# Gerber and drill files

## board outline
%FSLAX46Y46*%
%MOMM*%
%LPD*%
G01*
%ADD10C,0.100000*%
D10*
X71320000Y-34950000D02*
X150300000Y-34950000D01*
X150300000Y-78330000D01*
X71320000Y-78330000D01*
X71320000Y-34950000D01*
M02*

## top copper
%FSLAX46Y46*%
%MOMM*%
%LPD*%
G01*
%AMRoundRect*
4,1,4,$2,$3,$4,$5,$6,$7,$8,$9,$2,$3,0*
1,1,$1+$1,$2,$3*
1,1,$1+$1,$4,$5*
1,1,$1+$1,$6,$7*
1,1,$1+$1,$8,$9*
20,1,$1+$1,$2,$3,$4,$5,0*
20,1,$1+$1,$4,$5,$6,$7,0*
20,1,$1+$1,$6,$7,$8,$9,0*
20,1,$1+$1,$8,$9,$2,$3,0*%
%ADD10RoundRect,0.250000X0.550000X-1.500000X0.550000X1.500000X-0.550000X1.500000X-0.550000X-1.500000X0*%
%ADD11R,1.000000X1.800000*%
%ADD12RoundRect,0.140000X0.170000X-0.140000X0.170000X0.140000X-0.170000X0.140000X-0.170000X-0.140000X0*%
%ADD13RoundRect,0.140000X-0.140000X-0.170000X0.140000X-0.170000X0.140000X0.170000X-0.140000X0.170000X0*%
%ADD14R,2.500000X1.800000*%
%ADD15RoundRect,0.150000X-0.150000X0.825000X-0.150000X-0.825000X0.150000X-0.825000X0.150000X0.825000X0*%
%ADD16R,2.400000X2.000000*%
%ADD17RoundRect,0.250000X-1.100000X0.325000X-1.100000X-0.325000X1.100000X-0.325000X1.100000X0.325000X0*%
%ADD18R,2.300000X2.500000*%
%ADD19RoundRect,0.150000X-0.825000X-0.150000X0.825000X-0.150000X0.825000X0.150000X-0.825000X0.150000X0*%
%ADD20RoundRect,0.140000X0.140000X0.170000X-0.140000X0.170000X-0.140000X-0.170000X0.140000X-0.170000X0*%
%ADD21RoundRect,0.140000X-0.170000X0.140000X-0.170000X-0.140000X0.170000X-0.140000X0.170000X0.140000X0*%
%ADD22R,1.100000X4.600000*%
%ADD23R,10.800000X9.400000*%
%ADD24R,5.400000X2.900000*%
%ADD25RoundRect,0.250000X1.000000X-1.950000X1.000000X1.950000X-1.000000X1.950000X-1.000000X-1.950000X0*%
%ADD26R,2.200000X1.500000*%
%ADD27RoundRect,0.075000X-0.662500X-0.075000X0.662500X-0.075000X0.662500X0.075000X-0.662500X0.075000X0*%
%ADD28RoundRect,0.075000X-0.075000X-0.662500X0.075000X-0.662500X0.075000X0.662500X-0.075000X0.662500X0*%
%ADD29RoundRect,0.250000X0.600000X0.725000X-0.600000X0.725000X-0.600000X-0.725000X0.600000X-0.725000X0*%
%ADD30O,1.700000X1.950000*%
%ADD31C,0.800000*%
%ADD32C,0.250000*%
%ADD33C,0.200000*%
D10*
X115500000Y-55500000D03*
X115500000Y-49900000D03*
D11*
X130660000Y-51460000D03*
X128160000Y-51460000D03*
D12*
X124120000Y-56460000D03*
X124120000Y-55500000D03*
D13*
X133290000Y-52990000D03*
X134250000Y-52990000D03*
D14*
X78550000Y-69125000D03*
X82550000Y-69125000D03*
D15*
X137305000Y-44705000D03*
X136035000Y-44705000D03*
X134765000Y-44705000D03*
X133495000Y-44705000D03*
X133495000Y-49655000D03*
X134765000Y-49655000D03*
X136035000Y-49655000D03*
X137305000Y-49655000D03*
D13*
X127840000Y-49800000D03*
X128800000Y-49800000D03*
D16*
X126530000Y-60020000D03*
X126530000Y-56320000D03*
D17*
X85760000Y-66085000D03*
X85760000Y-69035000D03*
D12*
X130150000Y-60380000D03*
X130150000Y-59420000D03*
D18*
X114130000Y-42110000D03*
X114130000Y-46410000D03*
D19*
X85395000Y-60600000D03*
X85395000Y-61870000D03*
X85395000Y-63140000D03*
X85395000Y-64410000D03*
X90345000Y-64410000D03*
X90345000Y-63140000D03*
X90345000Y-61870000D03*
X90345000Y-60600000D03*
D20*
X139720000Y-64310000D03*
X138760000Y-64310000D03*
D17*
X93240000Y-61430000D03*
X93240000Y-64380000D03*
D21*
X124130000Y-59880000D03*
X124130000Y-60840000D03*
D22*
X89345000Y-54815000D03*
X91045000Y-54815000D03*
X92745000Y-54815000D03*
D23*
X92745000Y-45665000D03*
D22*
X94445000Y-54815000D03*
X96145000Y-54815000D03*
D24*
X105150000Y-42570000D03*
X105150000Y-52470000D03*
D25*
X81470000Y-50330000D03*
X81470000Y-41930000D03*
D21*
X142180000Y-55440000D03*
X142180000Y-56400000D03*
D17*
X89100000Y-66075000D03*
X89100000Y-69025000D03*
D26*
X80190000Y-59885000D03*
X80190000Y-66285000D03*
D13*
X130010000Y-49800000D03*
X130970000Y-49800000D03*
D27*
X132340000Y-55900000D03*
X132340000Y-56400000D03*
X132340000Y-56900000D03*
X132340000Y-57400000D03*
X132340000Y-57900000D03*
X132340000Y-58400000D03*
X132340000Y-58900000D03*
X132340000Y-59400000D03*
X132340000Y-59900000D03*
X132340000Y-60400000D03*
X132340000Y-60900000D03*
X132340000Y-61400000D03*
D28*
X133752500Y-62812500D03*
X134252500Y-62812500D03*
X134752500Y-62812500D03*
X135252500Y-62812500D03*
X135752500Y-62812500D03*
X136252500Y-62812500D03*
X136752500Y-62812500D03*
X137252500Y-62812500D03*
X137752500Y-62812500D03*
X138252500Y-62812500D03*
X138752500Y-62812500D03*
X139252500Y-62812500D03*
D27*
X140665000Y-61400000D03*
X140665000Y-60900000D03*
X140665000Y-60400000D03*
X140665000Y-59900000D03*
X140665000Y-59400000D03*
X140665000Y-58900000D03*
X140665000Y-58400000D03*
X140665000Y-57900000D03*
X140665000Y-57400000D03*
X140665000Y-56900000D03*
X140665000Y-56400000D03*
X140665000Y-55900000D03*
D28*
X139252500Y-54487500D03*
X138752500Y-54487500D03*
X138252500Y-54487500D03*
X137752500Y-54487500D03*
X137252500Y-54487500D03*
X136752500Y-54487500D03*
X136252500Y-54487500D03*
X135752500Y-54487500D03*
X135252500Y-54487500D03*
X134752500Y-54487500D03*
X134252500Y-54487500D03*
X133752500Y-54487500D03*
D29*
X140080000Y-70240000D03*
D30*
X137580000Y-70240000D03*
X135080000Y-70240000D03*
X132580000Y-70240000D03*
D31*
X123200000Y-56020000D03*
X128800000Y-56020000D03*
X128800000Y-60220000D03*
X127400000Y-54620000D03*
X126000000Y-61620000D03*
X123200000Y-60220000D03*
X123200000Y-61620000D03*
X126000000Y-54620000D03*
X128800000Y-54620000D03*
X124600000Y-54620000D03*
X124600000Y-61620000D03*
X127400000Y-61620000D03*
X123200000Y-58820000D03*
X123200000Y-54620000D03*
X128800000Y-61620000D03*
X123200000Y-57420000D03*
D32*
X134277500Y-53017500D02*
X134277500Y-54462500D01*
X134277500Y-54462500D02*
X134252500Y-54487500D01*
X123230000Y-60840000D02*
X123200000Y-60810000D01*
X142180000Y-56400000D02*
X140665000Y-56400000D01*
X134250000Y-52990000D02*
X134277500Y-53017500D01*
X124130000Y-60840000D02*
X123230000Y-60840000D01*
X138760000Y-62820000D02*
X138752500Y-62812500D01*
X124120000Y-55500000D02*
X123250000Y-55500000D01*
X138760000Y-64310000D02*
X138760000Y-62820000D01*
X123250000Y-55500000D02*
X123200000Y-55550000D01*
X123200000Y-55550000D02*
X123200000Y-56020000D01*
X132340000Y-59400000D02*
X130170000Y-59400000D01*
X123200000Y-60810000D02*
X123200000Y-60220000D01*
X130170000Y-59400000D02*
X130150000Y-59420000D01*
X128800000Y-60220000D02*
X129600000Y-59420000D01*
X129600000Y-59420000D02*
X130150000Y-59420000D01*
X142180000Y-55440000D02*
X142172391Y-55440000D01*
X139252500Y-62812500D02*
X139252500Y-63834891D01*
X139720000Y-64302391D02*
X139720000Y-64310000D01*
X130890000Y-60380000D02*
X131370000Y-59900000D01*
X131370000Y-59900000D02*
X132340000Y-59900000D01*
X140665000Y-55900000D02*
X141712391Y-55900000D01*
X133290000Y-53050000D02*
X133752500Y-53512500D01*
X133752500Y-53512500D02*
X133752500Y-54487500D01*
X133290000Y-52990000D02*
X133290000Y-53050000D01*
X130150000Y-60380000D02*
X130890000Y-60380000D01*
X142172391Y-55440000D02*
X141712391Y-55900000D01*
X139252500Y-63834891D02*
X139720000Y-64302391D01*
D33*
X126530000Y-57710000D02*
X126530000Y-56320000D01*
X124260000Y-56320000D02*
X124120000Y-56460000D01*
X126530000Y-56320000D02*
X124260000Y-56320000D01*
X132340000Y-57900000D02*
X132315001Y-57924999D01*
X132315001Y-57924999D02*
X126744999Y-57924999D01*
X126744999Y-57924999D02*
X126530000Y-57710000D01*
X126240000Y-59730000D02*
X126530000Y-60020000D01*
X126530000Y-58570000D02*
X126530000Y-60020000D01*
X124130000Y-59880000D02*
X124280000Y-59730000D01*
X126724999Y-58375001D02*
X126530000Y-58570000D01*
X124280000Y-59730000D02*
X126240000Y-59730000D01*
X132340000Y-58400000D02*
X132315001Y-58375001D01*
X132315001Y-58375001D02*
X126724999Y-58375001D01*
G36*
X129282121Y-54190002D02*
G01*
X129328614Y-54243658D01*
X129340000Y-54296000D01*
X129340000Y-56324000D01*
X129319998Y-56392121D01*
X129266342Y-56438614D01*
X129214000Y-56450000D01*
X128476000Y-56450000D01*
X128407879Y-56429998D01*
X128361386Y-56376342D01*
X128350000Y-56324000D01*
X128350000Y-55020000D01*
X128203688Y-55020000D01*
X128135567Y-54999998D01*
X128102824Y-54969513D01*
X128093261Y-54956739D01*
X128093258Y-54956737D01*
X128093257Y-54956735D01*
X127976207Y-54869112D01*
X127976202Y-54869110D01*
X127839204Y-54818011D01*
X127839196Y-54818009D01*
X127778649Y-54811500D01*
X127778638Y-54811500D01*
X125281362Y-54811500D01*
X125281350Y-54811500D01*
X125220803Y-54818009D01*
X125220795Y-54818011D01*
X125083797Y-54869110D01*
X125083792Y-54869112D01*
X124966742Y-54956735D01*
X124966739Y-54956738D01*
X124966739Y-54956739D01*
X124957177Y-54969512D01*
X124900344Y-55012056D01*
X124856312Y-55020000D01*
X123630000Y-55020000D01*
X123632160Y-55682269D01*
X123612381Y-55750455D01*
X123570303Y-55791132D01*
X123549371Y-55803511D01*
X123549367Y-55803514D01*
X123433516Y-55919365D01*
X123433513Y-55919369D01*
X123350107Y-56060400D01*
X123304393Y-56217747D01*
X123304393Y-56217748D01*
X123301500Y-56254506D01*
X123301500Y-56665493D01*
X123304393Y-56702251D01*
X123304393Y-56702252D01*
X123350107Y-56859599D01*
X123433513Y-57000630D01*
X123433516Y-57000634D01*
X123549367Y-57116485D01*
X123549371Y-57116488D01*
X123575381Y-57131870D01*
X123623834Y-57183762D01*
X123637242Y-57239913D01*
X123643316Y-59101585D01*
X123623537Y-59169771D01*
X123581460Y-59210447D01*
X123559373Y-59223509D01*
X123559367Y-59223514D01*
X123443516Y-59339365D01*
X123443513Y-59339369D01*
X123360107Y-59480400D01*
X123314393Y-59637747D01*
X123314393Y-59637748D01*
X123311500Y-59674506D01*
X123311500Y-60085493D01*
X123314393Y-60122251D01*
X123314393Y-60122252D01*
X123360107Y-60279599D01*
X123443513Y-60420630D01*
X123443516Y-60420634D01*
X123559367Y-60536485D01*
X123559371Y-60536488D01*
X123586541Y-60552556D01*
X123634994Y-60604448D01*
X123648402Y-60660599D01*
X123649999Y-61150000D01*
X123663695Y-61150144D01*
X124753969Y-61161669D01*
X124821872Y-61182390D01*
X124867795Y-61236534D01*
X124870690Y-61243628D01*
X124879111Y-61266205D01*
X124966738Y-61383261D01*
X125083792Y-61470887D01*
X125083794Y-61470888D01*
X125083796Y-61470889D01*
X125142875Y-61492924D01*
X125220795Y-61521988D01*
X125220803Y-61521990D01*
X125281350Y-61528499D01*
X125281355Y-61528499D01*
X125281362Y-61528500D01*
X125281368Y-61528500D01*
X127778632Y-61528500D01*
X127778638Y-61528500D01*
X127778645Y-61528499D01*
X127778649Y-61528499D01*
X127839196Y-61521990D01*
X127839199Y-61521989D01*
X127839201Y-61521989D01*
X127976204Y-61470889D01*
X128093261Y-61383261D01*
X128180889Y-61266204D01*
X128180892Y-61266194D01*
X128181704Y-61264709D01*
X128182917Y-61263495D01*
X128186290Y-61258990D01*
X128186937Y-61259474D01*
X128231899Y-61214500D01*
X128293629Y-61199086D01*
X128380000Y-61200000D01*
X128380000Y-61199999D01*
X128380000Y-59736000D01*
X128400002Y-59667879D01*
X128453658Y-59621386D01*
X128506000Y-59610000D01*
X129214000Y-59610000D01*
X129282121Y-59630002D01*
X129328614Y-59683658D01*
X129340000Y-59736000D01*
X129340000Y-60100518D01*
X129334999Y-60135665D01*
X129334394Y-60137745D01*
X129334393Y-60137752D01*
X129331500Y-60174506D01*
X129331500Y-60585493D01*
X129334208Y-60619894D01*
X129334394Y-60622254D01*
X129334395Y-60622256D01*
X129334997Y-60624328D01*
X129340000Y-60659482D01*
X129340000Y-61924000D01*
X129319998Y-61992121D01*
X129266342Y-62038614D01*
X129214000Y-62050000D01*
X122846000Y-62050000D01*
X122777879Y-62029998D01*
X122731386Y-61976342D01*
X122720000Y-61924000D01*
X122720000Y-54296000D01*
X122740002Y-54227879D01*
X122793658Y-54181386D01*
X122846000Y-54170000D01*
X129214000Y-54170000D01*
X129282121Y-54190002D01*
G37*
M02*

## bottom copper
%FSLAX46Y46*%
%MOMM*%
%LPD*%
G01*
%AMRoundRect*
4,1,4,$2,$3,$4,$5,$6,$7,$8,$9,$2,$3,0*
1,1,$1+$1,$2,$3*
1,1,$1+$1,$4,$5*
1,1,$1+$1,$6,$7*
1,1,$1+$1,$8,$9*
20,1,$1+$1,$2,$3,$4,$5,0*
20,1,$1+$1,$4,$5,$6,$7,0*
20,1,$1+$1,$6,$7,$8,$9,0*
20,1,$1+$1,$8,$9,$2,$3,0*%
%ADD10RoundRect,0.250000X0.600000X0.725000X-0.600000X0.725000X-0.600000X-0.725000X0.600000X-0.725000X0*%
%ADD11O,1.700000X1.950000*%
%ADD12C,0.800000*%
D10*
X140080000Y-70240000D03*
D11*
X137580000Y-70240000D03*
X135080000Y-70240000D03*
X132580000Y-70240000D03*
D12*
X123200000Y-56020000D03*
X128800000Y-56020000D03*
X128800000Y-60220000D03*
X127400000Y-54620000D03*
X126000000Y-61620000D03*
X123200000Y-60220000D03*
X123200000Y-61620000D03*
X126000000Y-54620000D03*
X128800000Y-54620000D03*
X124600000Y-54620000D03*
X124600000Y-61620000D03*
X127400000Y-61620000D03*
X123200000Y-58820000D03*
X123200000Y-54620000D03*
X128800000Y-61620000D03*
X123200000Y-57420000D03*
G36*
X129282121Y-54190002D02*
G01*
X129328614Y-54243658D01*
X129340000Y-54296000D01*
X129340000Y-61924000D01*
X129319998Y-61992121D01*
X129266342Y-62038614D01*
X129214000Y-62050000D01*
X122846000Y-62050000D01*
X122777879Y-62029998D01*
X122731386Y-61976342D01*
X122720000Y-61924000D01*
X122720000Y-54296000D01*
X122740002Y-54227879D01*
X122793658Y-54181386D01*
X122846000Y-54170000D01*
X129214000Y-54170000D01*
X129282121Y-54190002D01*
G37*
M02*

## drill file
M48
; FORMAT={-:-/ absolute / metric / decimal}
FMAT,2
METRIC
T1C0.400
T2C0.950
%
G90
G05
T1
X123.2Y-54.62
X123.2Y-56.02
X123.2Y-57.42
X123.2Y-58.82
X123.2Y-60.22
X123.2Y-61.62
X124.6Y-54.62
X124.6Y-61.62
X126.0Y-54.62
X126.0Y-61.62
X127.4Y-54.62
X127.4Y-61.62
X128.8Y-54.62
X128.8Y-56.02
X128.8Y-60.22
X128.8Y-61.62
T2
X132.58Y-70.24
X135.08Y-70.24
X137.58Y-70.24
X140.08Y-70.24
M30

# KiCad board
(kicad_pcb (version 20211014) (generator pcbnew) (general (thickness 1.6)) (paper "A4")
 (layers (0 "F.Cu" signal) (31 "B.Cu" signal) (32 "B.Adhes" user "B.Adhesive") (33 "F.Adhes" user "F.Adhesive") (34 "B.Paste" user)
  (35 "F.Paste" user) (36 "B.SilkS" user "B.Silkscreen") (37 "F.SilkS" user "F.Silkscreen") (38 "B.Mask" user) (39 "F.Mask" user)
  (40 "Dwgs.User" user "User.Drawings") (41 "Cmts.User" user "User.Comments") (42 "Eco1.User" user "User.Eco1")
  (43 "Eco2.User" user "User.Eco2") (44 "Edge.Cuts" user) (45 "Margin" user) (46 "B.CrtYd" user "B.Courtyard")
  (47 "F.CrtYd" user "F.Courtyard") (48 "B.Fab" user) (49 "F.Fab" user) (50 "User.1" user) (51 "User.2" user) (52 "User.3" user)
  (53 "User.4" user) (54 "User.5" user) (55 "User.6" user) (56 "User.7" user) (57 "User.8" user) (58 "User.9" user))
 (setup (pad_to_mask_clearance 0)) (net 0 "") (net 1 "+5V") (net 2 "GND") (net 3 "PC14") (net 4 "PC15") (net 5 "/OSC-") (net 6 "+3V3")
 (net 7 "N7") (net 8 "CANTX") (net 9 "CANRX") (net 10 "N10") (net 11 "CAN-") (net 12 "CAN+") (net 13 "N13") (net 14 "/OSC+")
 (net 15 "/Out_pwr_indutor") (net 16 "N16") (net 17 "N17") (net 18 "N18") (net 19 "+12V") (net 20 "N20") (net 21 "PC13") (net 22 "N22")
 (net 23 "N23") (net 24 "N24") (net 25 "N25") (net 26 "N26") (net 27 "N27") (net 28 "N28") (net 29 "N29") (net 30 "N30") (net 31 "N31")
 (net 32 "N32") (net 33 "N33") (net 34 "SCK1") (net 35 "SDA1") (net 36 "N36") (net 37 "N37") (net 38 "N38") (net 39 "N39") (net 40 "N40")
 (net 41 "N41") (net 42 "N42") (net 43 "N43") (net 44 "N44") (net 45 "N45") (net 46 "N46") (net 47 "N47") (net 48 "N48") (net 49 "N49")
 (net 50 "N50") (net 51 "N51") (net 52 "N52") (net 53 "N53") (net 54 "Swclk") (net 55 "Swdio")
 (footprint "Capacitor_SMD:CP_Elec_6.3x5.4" (layer "F.Cu") (at 115.5 52.7 90) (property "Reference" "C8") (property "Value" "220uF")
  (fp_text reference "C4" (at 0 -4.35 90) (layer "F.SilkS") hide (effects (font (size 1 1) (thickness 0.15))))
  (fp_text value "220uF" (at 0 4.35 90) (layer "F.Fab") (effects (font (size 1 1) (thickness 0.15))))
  (pad "1" smd roundrect (at -2.8 0 90) (size 3.5 1.6) (layers "F.Cu" "F.Paste" "F.Mask") (roundrect_rratio 0.15625) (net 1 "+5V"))
  (pad "2" smd roundrect (at 2.8 0 90) (size 3.5 1.6) (layers "F.Cu" "F.Paste" "F.Mask") (roundrect_rratio 0.15625) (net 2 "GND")))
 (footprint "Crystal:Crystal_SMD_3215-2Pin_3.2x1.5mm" (layer "F.Cu") (at 129.41 51.46)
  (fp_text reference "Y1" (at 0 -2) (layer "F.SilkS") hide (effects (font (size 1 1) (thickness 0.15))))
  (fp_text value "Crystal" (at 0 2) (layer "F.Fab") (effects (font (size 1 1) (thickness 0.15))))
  (pad "1" smd rect (at 1.25 0) (size 1 1.8) (layers "F.Cu" "F.Paste" "F.Mask") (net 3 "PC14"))
  (pad "2" smd rect (at -1.25 0) (size 1 1.8) (layers "F.Cu" "F.Paste" "F.Mask") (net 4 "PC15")))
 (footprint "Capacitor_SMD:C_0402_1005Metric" (layer "F.Cu") (at 124.12 55.98 90) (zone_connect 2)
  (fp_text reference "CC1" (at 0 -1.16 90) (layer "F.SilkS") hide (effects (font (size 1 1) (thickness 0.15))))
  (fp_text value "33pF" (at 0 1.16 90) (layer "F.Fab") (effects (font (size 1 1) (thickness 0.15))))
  (pad "1" smd roundrect (at -0.48 0 90) (size 0.56 0.62) (layers "F.Cu" "F.Paste" "F.Mask") (roundrect_rratio 0.25) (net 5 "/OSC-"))
  (pad "2" smd roundrect (at 0.48 0 90) (size 0.56 0.62) (layers "F.Cu" "F.Paste" "F.Mask") (roundrect_rratio 0.25) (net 2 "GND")))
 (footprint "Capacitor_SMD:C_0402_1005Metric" (layer "F.Cu") (at 133.77 52.99)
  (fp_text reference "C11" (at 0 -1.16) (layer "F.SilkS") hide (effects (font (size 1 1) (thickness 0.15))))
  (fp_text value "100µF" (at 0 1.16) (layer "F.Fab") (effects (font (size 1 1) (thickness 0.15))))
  (pad "1" smd roundrect (at -0.48 0) (size 0.56 0.62) (layers "F.Cu" "F.Paste" "F.Mask") (roundrect_rratio 0.25) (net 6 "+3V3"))
  (pad "2" smd roundrect (at 0.48 0) (size 0.56 0.62) (layers "F.Cu" "F.Paste" "F.Mask") (roundrect_rratio 0.25) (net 2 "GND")))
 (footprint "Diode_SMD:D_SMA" (layer "F.Cu") (at 80.55 69.125)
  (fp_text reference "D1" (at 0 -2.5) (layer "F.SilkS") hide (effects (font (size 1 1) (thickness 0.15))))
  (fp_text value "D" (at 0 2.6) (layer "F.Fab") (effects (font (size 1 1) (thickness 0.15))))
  (pad "1" smd rect (at -2 0) (size 2.5 1.8) (layers "F.Cu" "F.Paste" "F.Mask") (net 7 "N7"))
  (pad "2" smd rect (at 2 0) (size 2.5 1.8) (layers "F.Cu" "F.Paste" "F.Mask") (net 2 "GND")))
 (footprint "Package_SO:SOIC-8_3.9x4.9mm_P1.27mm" (layer "F.Cu") (at 135.4 47.18 -90)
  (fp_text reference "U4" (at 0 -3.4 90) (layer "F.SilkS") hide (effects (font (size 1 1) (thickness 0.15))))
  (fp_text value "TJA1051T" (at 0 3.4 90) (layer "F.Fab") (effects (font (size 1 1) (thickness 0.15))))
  (pad "1" smd roundrect (at -2.475 -1.905 270) (size 1.95 0.6) (layers "F.Cu" "F.Paste" "F.Mask") (roundrect_rratio 0.25) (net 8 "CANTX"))
  (pad "2" smd roundrect (at -2.475 -0.635 270) (size 1.95 0.6) (layers "F.Cu" "F.Paste" "F.Mask") (roundrect_rratio 0.25) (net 2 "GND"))
  (pad "3" smd roundrect (at -2.475 0.635 270) (size 1.95 0.6) (layers "F.Cu" "F.Paste" "F.Mask") (roundrect_rratio 0.25) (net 1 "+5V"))
  (pad "4" smd roundrect (at -2.475 1.905 270) (size 1.95 0.6) (layers "F.Cu" "F.Paste" "F.Mask") (roundrect_rratio 0.25) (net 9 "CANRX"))
  (pad "5" smd roundrect (at 2.475 1.905 270) (size 1.95 0.6) (layers "F.Cu" "F.Paste" "F.Mask") (roundrect_rratio 0.25) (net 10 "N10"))
  (pad "6" smd roundrect (at 2.475 0.635 270) (size 1.95 0.6) (layers "F.Cu" "F.Paste" "F.Mask") (roundrect_rratio 0.25) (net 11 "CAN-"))
  (pad "7" smd roundrect (at 2.475 -0.635 270) (size 1.95 0.6) (layers "F.Cu" "F.Paste" "F.Mask") (roundrect_rratio 0.25) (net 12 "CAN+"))
  (pad "8" smd roundrect (at 2.475 -1.905 270) (size 1.95 0.6) (layers "F.Cu" "F.Paste" "F.Mask") (roundrect_rratio 0.25) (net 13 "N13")))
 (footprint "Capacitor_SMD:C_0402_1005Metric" (layer "F.Cu") (at 128.32 49.8)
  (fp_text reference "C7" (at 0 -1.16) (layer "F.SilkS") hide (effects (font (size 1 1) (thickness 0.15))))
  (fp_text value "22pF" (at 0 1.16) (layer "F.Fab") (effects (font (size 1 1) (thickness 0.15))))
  (pad "1" smd roundrect (at -0.48 0) (size 0.56 0.62) (layers "F.Cu" "F.Paste" "F.Mask") (roundrect_rratio 0.25) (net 2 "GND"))
  (pad "2" smd roundrect (at 0.48 0) (size 0.56 0.62) (layers "F.Cu" "F.Paste" "F.Mask") (roundrect_rratio 0.25) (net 4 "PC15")))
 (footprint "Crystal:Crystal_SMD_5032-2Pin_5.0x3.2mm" (layer "F.Cu") (at 126.53 58.17 90) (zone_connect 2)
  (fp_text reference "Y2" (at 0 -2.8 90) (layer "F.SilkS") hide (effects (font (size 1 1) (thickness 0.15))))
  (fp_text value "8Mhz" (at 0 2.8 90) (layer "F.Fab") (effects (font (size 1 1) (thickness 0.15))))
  (pad "1" smd rect (at -1.85 0 90) (size 2 2.4) (layers "F.Cu" "F.Paste" "F.Mask") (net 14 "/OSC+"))
  (pad "2" smd rect (at 1.85 0 90) (size 2 2.4) (layers "F.Cu" "F.Paste" "F.Mask") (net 5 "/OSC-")))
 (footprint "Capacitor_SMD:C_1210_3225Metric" (layer "F.Cu") (at 85.76 67.56 -90)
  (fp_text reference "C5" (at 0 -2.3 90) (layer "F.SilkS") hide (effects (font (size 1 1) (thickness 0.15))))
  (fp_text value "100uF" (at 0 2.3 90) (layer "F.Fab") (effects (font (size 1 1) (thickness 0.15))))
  (pad "1" smd roundrect (at -1.475 0 270) (size 1.15 2.7) (layers "F.Cu" "F.Paste" "F.Mask") (roundrect_rratio 0.217391) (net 6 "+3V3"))
  (pad "2" smd roundrect (at 1.475 0 270) (size 1.15 2.7) (layers "F.Cu" "F.Paste" "F.Mask") (roundrect_rratio 0.217391) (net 2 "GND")))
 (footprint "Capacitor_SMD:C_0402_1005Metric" (layer "F.Cu") (at 130.15 59.9 90)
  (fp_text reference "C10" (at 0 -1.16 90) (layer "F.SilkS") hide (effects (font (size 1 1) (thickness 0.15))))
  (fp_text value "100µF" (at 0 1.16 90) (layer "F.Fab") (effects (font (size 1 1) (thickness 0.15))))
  (pad "1" smd roundrect (at -0.48 0 90) (size 0.56 0.62) (layers "F.Cu" "F.Paste" "F.Mask") (roundrect_rratio 0.25) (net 6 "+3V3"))
  (pad "2" smd roundrect (at 0.48 0 90) (size 0.56 0.62) (layers "F.Cu" "F.Paste" "F.Mask") (roundrect_rratio 0.25) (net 2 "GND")))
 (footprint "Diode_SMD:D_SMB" (layer "F.Cu") (at 114.13 44.26 -90) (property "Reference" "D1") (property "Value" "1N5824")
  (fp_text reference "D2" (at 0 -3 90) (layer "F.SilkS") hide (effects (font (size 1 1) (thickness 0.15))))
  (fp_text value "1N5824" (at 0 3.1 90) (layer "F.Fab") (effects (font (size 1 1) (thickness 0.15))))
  (pad "1" smd rect (at -2.15 0 270) (size 2.5 2.3) (layers "F.Cu" "F.Paste" "F.Mask") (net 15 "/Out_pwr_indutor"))
  (pad "2" smd rect (at 2.15 0 270) (size 2.5 2.3) (layers "F.Cu" "F.Paste" "F.Mask") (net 2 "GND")))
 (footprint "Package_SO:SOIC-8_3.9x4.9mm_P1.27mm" (layer "F.Cu") (at 87.87 62.505)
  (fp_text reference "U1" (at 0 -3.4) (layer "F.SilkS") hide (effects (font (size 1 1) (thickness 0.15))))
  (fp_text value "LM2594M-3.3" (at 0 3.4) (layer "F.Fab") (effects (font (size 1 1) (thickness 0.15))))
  (pad "1" smd roundrect (at -2.475 -1.905) (size 1.95 0.6) (layers "F.Cu" "F.Paste" "F.Mask") (roundrect_rratio 0.25) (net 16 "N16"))
  (pad "2" smd roundrect (at -2.475 -0.635) (size 1.95 0.6) (layers "F.Cu" "F.Paste" "F.Mask") (roundrect_rratio 0.25) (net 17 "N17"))
  (pad "3" smd roundrect (at -2.475 0.635) (size 1.95 0.6) (layers "F.Cu" "F.Paste" "F.Mask") (roundrect_rratio 0.25) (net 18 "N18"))
  (pad "4" smd roundrect (at -2.475 1.905) (size 1.95 0.6) (layers "F.Cu" "F.Paste" "F.Mask") (roundrect_rratio 0.25) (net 6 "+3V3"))
  (pad "5" smd roundrect (at 2.475 1.905) (size 1.95 0.6) (layers "F.Cu" "F.Paste" "F.Mask") (roundrect_rratio 0.25) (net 2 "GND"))
  (pad "6" smd roundrect (at 2.475 0.635) (size 1.95 0.6) (layers "F.Cu" "F.Paste" "F.Mask") (roundrect_rratio 0.25) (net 2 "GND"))
  (pad "7" smd roundrect (at 2.475 -0.635) (size 1.95 0.6) (layers "F.Cu" "F.Paste" "F.Mask") (roundrect_rratio 0.25) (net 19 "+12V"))
  (pad "8" smd roundrect (at 2.475 -1.905) (size 1.95 0.6) (layers "F.Cu" "F.Paste" "F.Mask") (roundrect_rratio 0.25) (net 7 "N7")))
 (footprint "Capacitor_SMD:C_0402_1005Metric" (layer "F.Cu") (at 139.24 64.31 180)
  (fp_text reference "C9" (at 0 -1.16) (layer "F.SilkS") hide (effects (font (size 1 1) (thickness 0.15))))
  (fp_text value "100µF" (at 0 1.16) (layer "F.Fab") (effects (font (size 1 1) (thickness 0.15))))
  (pad "1" smd roundrect (at -0.48 0 180) (size 0.56 0.62) (layers "F.Cu" "F.Paste" "F.Mask") (roundrect_rratio 0.25) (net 6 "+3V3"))
  (pad "2" smd roundrect (at 0.48 0 180) (size 0.56 0.62) (layers "F.Cu" "F.Paste" "F.Mask") (roundrect_rratio 0.25) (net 2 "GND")))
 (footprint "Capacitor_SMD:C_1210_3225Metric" (layer "F.Cu") (at 93.24 62.905 -90)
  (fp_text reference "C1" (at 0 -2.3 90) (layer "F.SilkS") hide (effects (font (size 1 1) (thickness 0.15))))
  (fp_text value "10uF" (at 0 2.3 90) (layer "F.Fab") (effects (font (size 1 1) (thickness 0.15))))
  (pad "1" smd roundrect (at -1.475 0 270) (size 1.15 2.7) (layers "F.Cu" "F.Paste" "F.Mask") (roundrect_rratio 0.217391) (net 19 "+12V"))
  (pad "2" smd roundrect (at 1.475 0 270) (size 1.15 2.7) (layers "F.Cu" "F.Paste" "F.Mask") (roundrect_rratio 0.217391) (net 2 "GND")))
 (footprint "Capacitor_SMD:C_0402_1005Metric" (layer "F.Cu") (at 124.13 60.36 -90) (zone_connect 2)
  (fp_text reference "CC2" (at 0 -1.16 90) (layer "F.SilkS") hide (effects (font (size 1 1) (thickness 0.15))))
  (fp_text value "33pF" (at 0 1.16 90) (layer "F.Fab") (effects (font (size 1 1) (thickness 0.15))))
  (pad "1" smd roundrect (at -0.48 0 270) (size 0.56 0.62) (layers "F.Cu" "F.Paste" "F.Mask") (roundrect_rratio 0.25) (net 14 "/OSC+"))
  (pad "2" smd roundrect (at 0.48 0 270) (size 0.56 0.62) (layers "F.Cu" "F.Paste" "F.Mask") (roundrect_rratio 0.25) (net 2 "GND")))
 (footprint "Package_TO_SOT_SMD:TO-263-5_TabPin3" (layer "F.Cu") (at 92.745 49.04 90)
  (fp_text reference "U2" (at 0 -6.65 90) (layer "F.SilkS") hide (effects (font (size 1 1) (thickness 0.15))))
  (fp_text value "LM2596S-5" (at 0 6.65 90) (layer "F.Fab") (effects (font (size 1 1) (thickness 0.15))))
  (pad "" smd rect (at 0.95 -2.775 90) (size 4.55 5.25) (layers "F.Paste"))
  (pad "" smd rect (at 5.8 2.775 90) (size 4.55 5.25) (layers "F.Paste"))
  (pad "" smd rect (at 0.95 2.775 90) (size 4.55 5.25) (layers "F.Paste"))
  (pad "" smd rect (at 5.8 -2.775 90) (size 4.55 5.25) (layers "F.Paste"))
  (pad "1" smd rect (at -5.775 -3.4 90) (size 4.6 1.1) (layers "F.Cu" "F.Paste" "F.Mask") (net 19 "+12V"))
  (pad "2" smd rect (at -5.775 -1.7 90) (size 4.6 1.1) (layers "F.Cu" "F.Paste" "F.Mask") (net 15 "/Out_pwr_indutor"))
  (pad "3" smd rect (at -5.775 0 90) (size 4.6 1.1) (layers "F.Cu" "F.Paste" "F.Mask") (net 2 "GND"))
  (pad "3" smd rect (at 3.375 0 90) (size 9.4 10.8) (layers "F.Cu" "F.Mask") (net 2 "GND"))
  (pad "4" smd rect (at -5.775 1.7 90) (size 4.6 1.1) (layers "F.Cu" "F.Paste" "F.Mask") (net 1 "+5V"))
  (pad "5" smd rect (at -5.775 3.4 90) (size 4.6 1.1) (layers "F.Cu" "F.Paste" "F.Mask") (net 2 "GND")))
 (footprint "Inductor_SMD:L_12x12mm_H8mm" (layer "F.Cu") (at 105.15 47.52 -90)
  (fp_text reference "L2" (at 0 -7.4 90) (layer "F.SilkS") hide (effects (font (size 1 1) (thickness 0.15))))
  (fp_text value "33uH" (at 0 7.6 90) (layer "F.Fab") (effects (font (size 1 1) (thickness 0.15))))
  (pad "1" smd rect (at -4.95 0 270) (size 2.9 5.4) (layers "F.Cu" "F.Paste" "F.Mask") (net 15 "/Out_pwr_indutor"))
  (pad "2" smd rect (at 4.95 0 270) (size 2.9 5.4) (layers "F.Cu" "F.Paste" "F.Mask") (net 1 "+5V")))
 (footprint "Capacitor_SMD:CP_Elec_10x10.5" (layer "F.Cu") (at 81.47 46.13 90) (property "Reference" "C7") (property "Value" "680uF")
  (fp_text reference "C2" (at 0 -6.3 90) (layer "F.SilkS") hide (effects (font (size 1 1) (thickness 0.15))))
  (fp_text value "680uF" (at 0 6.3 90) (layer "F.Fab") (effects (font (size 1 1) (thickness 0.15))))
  (pad "1" smd roundrect (at -4.2 0 90) (size 4.4 2.5) (layers "F.Cu" "F.Paste" "F.Mask") (roundrect_rratio 0.1) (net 19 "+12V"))
  (pad "2" smd roundrect (at 4.2 0 90) (size 4.4 2.5) (layers "F.Cu" "F.Paste" "F.Mask") (roundrect_rratio 0.1) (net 2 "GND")))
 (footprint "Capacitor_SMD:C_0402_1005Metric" (layer "F.Cu") (at 142.18 55.92 -90)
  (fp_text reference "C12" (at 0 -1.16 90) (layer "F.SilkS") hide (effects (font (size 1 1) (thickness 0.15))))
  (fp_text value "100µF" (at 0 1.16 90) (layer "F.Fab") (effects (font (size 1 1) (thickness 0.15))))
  (pad "1" smd roundrect (at -0.48 0 270) (size 0.56 0.62) (layers "F.Cu" "F.Paste" "F.Mask") (roundrect_rratio 0.25) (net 6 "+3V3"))
  (pad "2" smd roundrect (at 0.48 0 270) (size 0.56 0.62) (layers "F.Cu" "F.Paste" "F.Mask") (roundrect_rratio 0.25) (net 2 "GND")))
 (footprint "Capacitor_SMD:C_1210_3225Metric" (layer "F.Cu") (at 89.1 67.55 -90)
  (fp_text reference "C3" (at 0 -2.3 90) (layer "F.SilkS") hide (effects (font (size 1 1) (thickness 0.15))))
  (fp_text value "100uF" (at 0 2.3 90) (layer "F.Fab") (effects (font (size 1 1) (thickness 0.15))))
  (pad "1" smd roundrect (at -1.475 0 270) (size 1.15 2.7) (layers "F.Cu" "F.Paste" "F.Mask") (roundrect_rratio 0.217391) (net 6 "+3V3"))
  (pad "2" smd roundrect (at 1.475 0 270) (size 1.15 2.7) (layers "F.Cu" "F.Paste" "F.Mask") (roundrect_rratio 0.217391) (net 2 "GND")))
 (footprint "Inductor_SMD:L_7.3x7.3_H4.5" (layer "F.Cu") (at 80.19 63.085 -90)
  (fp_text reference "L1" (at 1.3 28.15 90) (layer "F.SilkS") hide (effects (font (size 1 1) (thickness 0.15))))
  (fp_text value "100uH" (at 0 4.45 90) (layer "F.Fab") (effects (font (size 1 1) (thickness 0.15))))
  (pad "1" smd rect (at -3.2 0 270) (size 1.5 2.2) (layers "F.Cu" "F.Paste" "F.Mask") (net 7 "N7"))
  (pad "2" smd rect (at 3.2 0 270) (size 1.5 2.2) (layers "F.Cu" "F.Paste" "F.Mask") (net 6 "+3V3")))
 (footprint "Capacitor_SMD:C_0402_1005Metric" (layer "F.Cu") (at 130.49 49.8)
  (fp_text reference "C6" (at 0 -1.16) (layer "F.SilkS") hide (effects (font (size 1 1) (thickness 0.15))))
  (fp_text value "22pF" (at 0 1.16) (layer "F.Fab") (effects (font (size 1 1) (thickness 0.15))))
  (pad "1" smd roundrect (at -0.48 0) (size 0.56 0.62) (layers "F.Cu" "F.Paste" "F.Mask") (roundrect_rratio 0.25) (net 3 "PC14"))
  (pad "2" smd roundrect (at 0.48 0) (size 0.56 0.62) (layers "F.Cu" "F.Paste" "F.Mask") (roundrect_rratio 0.25) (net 2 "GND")))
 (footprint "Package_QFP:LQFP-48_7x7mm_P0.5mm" (layer "F.Cu") (at 136.5025 58.65)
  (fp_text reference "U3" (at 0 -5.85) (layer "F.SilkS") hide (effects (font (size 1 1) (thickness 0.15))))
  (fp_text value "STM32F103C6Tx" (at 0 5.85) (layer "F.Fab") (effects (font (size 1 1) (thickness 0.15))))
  (pad "1" smd roundrect (at -4.1625 -2.75) (size 1.475 0.3) (layers "F.Cu" "F.Paste" "F.Mask") (roundrect_rratio 0.25) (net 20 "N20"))
  (pad "2" smd roundrect (at -4.1625 -2.25) (size 1.475 0.3) (layers "F.Cu" "F.Paste" "F.Mask") (roundrect_rratio 0.25) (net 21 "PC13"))
  (pad "3" smd roundrect (at -4.1625 -1.75) (size 1.475 0.3) (layers "F.Cu" "F.Paste" "F.Mask") (roundrect_rratio 0.25) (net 3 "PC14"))
  (pad "4" smd roundrect (at -4.1625 -1.25) (size 1.475 0.3) (layers "F.Cu" "F.Paste" "F.Mask") (roundrect_rratio 0.25) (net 4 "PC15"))
  (pad "5" smd roundrect (at -4.1625 -0.75) (size 1.475 0.3) (layers "F.Cu" "F.Paste" "F.Mask") (roundrect_rratio 0.25) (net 5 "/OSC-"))
  (pad "6" smd roundrect (at -4.1625 -0.25) (size 1.475 0.3) (layers "F.Cu" "F.Paste" "F.Mask") (roundrect_rratio 0.25) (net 14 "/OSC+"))
  (pad "7" smd roundrect (at -4.1625 0.25) (size 1.475 0.3) (layers "F.Cu" "F.Paste" "F.Mask") (roundrect_rratio 0.25) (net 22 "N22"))
  (pad "8" smd roundrect (at -4.1625 0.75) (size 1.475 0.3) (layers "F.Cu" "F.Paste" "F.Mask") (roundrect_rratio 0.25) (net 2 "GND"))
  (pad "9" smd roundrect (at -4.1625 1.25) (size 1.475 0.3) (layers "F.Cu" "F.Paste" "F.Mask") (roundrect_rratio 0.25) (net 6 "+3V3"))
  (pad "10" smd roundrect (at -4.1625 1.75) (size 1.475 0.3) (layers "F.Cu" "F.Paste" "F.Mask") (roundrect_rratio 0.25) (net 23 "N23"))
  (pad "11" smd roundrect (at -4.1625 2.25) (size 1.475 0.3) (layers "F.Cu" "F.Paste" "F.Mask") (roundrect_rratio 0.25) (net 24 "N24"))
  (pad "12" smd roundrect (at -4.1625 2.75) (size 1.475 0.3) (layers "F.Cu" "F.Paste" "F.Mask") (roundrect_rratio 0.25) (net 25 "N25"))
  (pad "13" smd roundrect (at -2.75 4.1625) (size 0.3 1.475) (layers "F.Cu" "F.Paste" "F.Mask") (roundrect_rratio 0.25) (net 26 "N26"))
  (pad "14" smd roundrect (at -2.25 4.1625) (size 0.3 1.475) (layers "F.Cu" "F.Paste" "F.Mask") (roundrect_rratio 0.25) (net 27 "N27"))
  (pad "15" smd roundrect (at -1.75 4.1625) (size 0.3 1.475) (layers "F.Cu" "F.Paste" "F.Mask") (roundrect_rratio 0.25) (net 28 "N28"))
  (pad "16" smd roundrect (at -1.25 4.1625) (size 0.3 1.475) (layers "F.Cu" "F.Paste" "F.Mask") (roundrect_rratio 0.25) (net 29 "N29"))
  (pad "17" smd roundrect (at -0.75 4.1625) (size 0.3 1.475) (layers "F.Cu" "F.Paste" "F.Mask") (roundrect_rratio 0.25) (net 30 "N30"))
  (pad "18" smd roundrect (at -0.25 4.1625) (size 0.3 1.475) (layers "F.Cu" "F.Paste" "F.Mask") (roundrect_rratio 0.25) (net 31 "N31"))
  (pad "19" smd roundrect (at 0.25 4.1625) (size 0.3 1.475) (layers "F.Cu" "F.Paste" "F.Mask") (roundrect_rratio 0.25) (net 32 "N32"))
  (pad "20" smd roundrect (at 0.75 4.1625) (size 0.3 1.475) (layers "F.Cu" "F.Paste" "F.Mask") (roundrect_rratio 0.25) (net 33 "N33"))
  (pad "21" smd roundrect (at 1.25 4.1625) (size 0.3 1.475) (layers "F.Cu" "F.Paste" "F.Mask") (roundrect_rratio 0.25) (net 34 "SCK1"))
  (pad "22" smd roundrect (at 1.75 4.1625) (size 0.3 1.475) (layers "F.Cu" "F.Paste" "F.Mask") (roundrect_rratio 0.25) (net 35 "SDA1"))
  (pad "23" smd roundrect (at 2.25 4.1625) (size 0.3 1.475) (layers "F.Cu" "F.Paste" "F.Mask") (roundrect_rratio 0.25) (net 2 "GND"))
  (pad "24" smd roundrect (at 2.75 4.1625) (size 0.3 1.475) (layers "F.Cu" "F.Paste" "F.Mask") (roundrect_rratio 0.25) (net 6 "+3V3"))
  (pad "25" smd roundrect (at 4.1625 2.75) (size 1.475 0.3) (layers "F.Cu" "F.Paste" "F.Mask") (roundrect_rratio 0.25) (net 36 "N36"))
  (pad "26" smd roundrect (at 4.1625 2.25) (size 1.475 0.3) (layers "F.Cu" "F.Paste" "F.Mask") (roundrect_rratio 0.25) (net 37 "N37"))
  (pad "27" smd roundrect (at 4.1625 1.75) (size 1.475 0.3) (layers "F.Cu" "F.Paste" "F.Mask") (roundrect_rratio 0.25) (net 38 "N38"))
  (pad "28" smd roundrect (at 4.1625 1.25) (size 1.475 0.3) (layers "F.Cu" "F.Paste" "F.Mask") (roundrect_rratio 0.25) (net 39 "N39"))
  (pad "29" smd roundrect (at 4.1625 0.75) (size 1.475 0.3) (layers "F.Cu" "F.Paste" "F.Mask") (roundrect_rratio 0.25) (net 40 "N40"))
  (pad "30" smd roundrect (at 4.1625 0.25) (size 1.475 0.3) (layers "F.Cu" "F.Paste" "F.Mask") (roundrect_rratio 0.25) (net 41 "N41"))
  (pad "31" smd roundrect (at 4.1625 -0.25) (size 1.475 0.3) (layers "F.Cu" "F.Paste" "F.Mask") (roundrect_rratio 0.25) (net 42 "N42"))
  (pad "32" smd roundrect (at 4.1625 -0.75) (size 1.475 0.3) (layers "F.Cu" "F.Paste" "F.Mask") (roundrect_rratio 0.25) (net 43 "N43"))
  (pad "33" smd roundrect (at 4.1625 -1.25) (size 1.475 0.3) (layers "F.Cu" "F.Paste" "F.Mask") (roundrect_rratio 0.25) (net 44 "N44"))
  (pad "34" smd roundrect (at 4.1625 -1.75) (size 1.475 0.3) (layers "F.Cu" "F.Paste" "F.Mask") (roundrect_rratio 0.25) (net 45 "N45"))
  (pad "35" smd roundrect (at 4.1625 -2.25) (size 1.475 0.3) (layers "F.Cu" "F.Paste" "F.Mask") (roundrect_rratio 0.25) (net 2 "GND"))
  (pad "36" smd roundrect (at 4.1625 -2.75) (size 1.475 0.3) (layers "F.Cu" "F.Paste" "F.Mask") (roundrect_rratio 0.25) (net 6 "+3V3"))
  (pad "37" smd roundrect (at 2.75 -4.1625) (size 0.3 1.475) (layers "F.Cu" "F.Paste" "F.Mask") (roundrect_rratio 0.25) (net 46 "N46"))
  (pad "38" smd roundrect (at 2.25 -4.1625) (size 0.3 1.475) (layers "F.Cu" "F.Paste" "F.Mask") (roundrect_rratio 0.25) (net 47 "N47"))
  (pad "39" smd roundrect (at 1.75 -4.1625) (size 0.3 1.475) (layers "F.Cu" "F.Paste" "F.Mask") (roundrect_rratio 0.25) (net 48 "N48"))
  (pad "40" smd roundrect (at 1.25 -4.1625) (size 0.3 1.475) (layers "F.Cu" "F.Paste" "F.Mask") (roundrect_rratio 0.25) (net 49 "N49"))
  (pad "41" smd roundrect (at 0.75 -4.1625) (size 0.3 1.475) (layers "F.Cu" "F.Paste" "F.Mask") (roundrect_rratio 0.25) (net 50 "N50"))
  (pad "42" smd roundrect (at 0.25 -4.1625) (size 0.3 1.475) (layers "F.Cu" "F.Paste" "F.Mask") (roundrect_rratio 0.25) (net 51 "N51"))
  (pad "43" smd roundrect (at -0.25 -4.1625) (size 0.3 1.475) (layers "F.Cu" "F.Paste" "F.Mask") (roundrect_rratio 0.25) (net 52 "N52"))
  (pad "44" smd roundrect (at -0.75 -4.1625) (size 0.3 1.475) (layers "F.Cu" "F.Paste" "F.Mask") (roundrect_rratio 0.25) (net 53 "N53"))
  (pad "45" smd roundrect (at -1.25 -4.1625) (size 0.3 1.475) (layers "F.Cu" "F.Paste" "F.Mask") (roundrect_rratio 0.25) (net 9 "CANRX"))
  (pad "46" smd roundrect (at -1.75 -4.1625) (size 0.3 1.475) (layers "F.Cu" "F.Paste" "F.Mask") (roundrect_rratio 0.25) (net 8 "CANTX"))
  (pad "47" smd roundrect (at -2.25 -4.1625) (size 0.3 1.475) (layers "F.Cu" "F.Paste" "F.Mask") (roundrect_rratio 0.25) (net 2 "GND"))
  (pad "48" smd roundrect (at -2.75 -4.1625) (size 0.3 1.475) (layers "F.Cu" "F.Paste" "F.Mask") (roundrect_rratio 0.25) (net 6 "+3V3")))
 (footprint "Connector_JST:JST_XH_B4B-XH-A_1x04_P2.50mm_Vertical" (layer "F.Cu") (at 140.08 70.24 180)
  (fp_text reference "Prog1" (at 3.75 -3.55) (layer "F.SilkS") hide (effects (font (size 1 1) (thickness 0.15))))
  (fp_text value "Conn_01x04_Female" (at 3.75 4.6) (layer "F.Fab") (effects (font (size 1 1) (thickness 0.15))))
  (pad "1" thru_hole roundrect (at 0 0 180) (size 1.7 1.95) (drill 0.95) (layers *.Cu *.Mask) (roundrect_rratio 0.147059) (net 6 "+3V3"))
  (pad "2" thru_hole oval (at 2.5 0 180) (size 1.7 1.95) (drill 0.95) (layers *.Cu *.Mask) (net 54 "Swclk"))
  (pad "3" thru_hole oval (at 5 0 180) (size 1.7 1.95) (drill 0.95) (layers *.Cu *.Mask) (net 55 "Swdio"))
  (pad "4" thru_hole oval (at 7.5 0 180) (size 1.7 1.95) (drill 0.95) (layers *.Cu *.Mask) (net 2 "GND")))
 (gr_rect (start 71.32 34.95) (end 150.3 78.33) (layer "Edge.Cuts") (width 0.1) (fill none))
 (segment (start 134.2775 53.0175) (end 134.2775 54.4625) (width 0.25) (layer "F.Cu") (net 2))
 (segment (start 134.2775 54.4625) (end 134.2525 54.4875) (width 0.25) (layer "F.Cu") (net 2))
 (segment (start 123.23 60.84) (end 123.2 60.81) (width 0.25) (layer "F.Cu") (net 2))
 (segment (start 142.18 56.4) (end 140.665 56.4) (width 0.25) (layer "F.Cu") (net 2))
 (segment (start 134.25 52.99) (end 134.2775 53.0175) (width 0.25) (layer "F.Cu") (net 2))
 (segment (start 124.13 60.84) (end 123.23 60.84) (width 0.25) (layer "F.Cu") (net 2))
 (segment (start 138.76 62.82) (end 138.7525 62.8125) (width 0.25) (layer "F.Cu") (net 2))
 (segment (start 124.12 55.5) (end 123.25 55.5) (width 0.25) (layer "F.Cu") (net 2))
 (segment (start 138.76 64.31) (end 138.76 62.82) (width 0.25) (layer "F.Cu") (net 2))
 (segment (start 123.25 55.5) (end 123.2 55.55) (width 0.25) (layer "F.Cu") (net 2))
 (segment (start 123.2 55.55) (end 123.2 56.02) (width 0.25) (layer "F.Cu") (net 2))
 (segment (start 132.34 59.4) (end 130.17 59.4) (width 0.25) (layer "F.Cu") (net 2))
 (segment (start 123.2 60.81) (end 123.2 60.22) (width 0.25) (layer "F.Cu") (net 2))
 (segment (start 130.17 59.4) (end 130.15 59.42) (width 0.25) (layer "F.Cu") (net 2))
 (segment (start 128.8 60.22) (end 129.6 59.42) (width 0.25) (layer "F.Cu") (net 2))
 (segment (start 129.6 59.42) (end 130.15 59.42) (width 0.25) (layer "F.Cu") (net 2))
 (via (at 123.2 56.02) (size 0.8) (drill 0.4) (layers "F.Cu" "B.Cu") (free) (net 2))
 (via (at 128.8 56.02) (size 0.8) (drill 0.4) (layers "F.Cu" "B.Cu") (free) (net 2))
 (via (at 128.8 60.22) (size 0.8) (drill 0.4) (layers "F.Cu" "B.Cu") (free) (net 2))
 (via (at 127.4 54.62) (size 0.8) (drill 0.4) (layers "F.Cu" "B.Cu") (free) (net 2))
 (via (at 126 61.62) (size 0.8) (drill 0.4) (layers "F.Cu" "B.Cu") (free) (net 2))
 (via (at 123.2 60.22) (size 0.8) (drill 0.4) (layers "F.Cu" "B.Cu") (free) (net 2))
 (via (at 123.2 61.62) (size 0.8) (drill 0.4) (layers "F.Cu" "B.Cu") (free) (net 2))
 (via (at 126 54.62) (size 0.8) (drill 0.4) (layers "F.Cu" "B.Cu") (free) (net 2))
 (via (at 128.8 54.62) (size 0.8) (drill 0.4) (layers "F.Cu" "B.Cu") (free) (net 2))
 (via (at 124.6 54.62) (size 0.8) (drill 0.4) (layers "F.Cu" "B.Cu") (free) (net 2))
 (via (at 124.6 61.62) (size 0.8) (drill 0.4) (layers "F.Cu" "B.Cu") (free) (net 2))
 (via (at 127.4 61.62) (size 0.8) (drill 0.4) (layers "F.Cu" "B.Cu") (free) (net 2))
 (via (at 123.2 58.82) (size 0.8) (drill 0.4) (layers "F.Cu" "B.Cu") (free) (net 2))
 (via (at 123.2 54.62) (size 0.8) (drill 0.4) (layers "F.Cu" "B.Cu") (free) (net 2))
 (via (at 128.8 61.62) (size 0.8) (drill 0.4) (layers "F.Cu" "B.Cu") (free) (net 2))
 (via (at 123.2 57.42) (size 0.8) (drill 0.4) (layers "F.Cu" "B.Cu") (free) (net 2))
 (segment (start 142.18 55.44) (end 142.172391 55.44) (width 0.25) (layer "F.Cu") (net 6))
 (segment (start 139.2525 62.8125) (end 139.2525 63.834891) (width 0.25) (layer "F.Cu") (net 6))
 (segment (start 139.72 64.302391) (end 139.72 64.31) (width 0.25) (layer "F.Cu") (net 6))
 (segment (start 130.89 60.38) (end 131.37 59.9) (width 0.25) (layer "F.Cu") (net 6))
 (segment (start 131.37 59.9) (end 132.34 59.9) (width 0.25) (layer "F.Cu") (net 6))
 (segment (start 140.665 55.9) (end 141.712391 55.9) (width 0.25) (layer "F.Cu") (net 6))
 (segment (start 133.29 53.05) (end 133.7525 53.5125) (width 0.25) (layer "F.Cu") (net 6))
 (segment (start 133.7525 53.5125) (end 133.7525 54.4875) (width 0.25) (layer "F.Cu") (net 6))
 (segment (start 133.29 52.99) (end 133.29 53.05) (width 0.25) (layer "F.Cu") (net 6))
 (segment (start 130.15 60.38) (end 130.89 60.38) (width 0.25) (layer "F.Cu") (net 6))
 (segment (start 142.172391 55.44) (end 141.712391 55.9) (width 0.25) (layer "F.Cu") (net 6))
 (segment (start 139.2525 63.834891) (end 139.72 64.302391) (width 0.25) (layer "F.Cu") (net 6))
 (segment (start 126.53 57.71) (end 126.53 56.32) (width 0.2) (layer "F.Cu") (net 5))
 (segment (start 124.26 56.32) (end 124.12 56.46) (width 0.2) (layer "F.Cu") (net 5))
 (segment (start 126.53 56.32) (end 124.26 56.32) (width 0.2) (layer "F.Cu") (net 5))
 (segment (start 132.34 57.9) (end 132.315001 57.924999) (width 0.2) (layer "F.Cu") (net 5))
 (segment (start 132.315001 57.924999) (end 126.744999 57.924999) (width 0.2) (layer "F.Cu") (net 5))
 (segment (start 126.744999 57.924999) (end 126.53 57.71) (width 0.2) (layer "F.Cu") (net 5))
 (segment (start 126.24 59.73) (end 126.53 60.02) (width 0.2) (layer "F.Cu") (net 14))
 (segment (start 126.53 58.57) (end 126.53 60.02) (width 0.2) (layer "F.Cu") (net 14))
 (segment (start 124.13 59.88) (end 124.28 59.73) (width 0.2) (layer "F.Cu") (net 14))
 (segment (start 126.724999 58.375001) (end 126.53 58.57) (width 0.2) (layer "F.Cu") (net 14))
 (segment (start 124.28 59.73) (end 126.24 59.73) (width 0.2) (layer "F.Cu") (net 14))
 (segment (start 132.34 58.4) (end 132.315001 58.375001) (width 0.2) (layer "F.Cu") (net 14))
 (segment (start 132.315001 58.375001) (end 126.724999 58.375001) (width 0.2) (layer "F.Cu") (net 14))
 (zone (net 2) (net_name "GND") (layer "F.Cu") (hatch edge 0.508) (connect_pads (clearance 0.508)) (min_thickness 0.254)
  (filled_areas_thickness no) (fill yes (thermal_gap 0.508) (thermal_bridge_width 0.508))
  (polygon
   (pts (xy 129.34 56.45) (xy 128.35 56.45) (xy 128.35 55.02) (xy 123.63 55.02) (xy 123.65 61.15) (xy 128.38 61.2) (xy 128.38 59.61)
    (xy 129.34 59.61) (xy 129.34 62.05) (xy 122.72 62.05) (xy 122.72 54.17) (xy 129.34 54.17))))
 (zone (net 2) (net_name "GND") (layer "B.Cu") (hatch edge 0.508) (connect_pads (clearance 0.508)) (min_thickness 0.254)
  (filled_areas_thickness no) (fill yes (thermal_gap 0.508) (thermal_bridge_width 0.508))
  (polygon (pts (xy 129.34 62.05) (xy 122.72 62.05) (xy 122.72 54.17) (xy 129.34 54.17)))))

